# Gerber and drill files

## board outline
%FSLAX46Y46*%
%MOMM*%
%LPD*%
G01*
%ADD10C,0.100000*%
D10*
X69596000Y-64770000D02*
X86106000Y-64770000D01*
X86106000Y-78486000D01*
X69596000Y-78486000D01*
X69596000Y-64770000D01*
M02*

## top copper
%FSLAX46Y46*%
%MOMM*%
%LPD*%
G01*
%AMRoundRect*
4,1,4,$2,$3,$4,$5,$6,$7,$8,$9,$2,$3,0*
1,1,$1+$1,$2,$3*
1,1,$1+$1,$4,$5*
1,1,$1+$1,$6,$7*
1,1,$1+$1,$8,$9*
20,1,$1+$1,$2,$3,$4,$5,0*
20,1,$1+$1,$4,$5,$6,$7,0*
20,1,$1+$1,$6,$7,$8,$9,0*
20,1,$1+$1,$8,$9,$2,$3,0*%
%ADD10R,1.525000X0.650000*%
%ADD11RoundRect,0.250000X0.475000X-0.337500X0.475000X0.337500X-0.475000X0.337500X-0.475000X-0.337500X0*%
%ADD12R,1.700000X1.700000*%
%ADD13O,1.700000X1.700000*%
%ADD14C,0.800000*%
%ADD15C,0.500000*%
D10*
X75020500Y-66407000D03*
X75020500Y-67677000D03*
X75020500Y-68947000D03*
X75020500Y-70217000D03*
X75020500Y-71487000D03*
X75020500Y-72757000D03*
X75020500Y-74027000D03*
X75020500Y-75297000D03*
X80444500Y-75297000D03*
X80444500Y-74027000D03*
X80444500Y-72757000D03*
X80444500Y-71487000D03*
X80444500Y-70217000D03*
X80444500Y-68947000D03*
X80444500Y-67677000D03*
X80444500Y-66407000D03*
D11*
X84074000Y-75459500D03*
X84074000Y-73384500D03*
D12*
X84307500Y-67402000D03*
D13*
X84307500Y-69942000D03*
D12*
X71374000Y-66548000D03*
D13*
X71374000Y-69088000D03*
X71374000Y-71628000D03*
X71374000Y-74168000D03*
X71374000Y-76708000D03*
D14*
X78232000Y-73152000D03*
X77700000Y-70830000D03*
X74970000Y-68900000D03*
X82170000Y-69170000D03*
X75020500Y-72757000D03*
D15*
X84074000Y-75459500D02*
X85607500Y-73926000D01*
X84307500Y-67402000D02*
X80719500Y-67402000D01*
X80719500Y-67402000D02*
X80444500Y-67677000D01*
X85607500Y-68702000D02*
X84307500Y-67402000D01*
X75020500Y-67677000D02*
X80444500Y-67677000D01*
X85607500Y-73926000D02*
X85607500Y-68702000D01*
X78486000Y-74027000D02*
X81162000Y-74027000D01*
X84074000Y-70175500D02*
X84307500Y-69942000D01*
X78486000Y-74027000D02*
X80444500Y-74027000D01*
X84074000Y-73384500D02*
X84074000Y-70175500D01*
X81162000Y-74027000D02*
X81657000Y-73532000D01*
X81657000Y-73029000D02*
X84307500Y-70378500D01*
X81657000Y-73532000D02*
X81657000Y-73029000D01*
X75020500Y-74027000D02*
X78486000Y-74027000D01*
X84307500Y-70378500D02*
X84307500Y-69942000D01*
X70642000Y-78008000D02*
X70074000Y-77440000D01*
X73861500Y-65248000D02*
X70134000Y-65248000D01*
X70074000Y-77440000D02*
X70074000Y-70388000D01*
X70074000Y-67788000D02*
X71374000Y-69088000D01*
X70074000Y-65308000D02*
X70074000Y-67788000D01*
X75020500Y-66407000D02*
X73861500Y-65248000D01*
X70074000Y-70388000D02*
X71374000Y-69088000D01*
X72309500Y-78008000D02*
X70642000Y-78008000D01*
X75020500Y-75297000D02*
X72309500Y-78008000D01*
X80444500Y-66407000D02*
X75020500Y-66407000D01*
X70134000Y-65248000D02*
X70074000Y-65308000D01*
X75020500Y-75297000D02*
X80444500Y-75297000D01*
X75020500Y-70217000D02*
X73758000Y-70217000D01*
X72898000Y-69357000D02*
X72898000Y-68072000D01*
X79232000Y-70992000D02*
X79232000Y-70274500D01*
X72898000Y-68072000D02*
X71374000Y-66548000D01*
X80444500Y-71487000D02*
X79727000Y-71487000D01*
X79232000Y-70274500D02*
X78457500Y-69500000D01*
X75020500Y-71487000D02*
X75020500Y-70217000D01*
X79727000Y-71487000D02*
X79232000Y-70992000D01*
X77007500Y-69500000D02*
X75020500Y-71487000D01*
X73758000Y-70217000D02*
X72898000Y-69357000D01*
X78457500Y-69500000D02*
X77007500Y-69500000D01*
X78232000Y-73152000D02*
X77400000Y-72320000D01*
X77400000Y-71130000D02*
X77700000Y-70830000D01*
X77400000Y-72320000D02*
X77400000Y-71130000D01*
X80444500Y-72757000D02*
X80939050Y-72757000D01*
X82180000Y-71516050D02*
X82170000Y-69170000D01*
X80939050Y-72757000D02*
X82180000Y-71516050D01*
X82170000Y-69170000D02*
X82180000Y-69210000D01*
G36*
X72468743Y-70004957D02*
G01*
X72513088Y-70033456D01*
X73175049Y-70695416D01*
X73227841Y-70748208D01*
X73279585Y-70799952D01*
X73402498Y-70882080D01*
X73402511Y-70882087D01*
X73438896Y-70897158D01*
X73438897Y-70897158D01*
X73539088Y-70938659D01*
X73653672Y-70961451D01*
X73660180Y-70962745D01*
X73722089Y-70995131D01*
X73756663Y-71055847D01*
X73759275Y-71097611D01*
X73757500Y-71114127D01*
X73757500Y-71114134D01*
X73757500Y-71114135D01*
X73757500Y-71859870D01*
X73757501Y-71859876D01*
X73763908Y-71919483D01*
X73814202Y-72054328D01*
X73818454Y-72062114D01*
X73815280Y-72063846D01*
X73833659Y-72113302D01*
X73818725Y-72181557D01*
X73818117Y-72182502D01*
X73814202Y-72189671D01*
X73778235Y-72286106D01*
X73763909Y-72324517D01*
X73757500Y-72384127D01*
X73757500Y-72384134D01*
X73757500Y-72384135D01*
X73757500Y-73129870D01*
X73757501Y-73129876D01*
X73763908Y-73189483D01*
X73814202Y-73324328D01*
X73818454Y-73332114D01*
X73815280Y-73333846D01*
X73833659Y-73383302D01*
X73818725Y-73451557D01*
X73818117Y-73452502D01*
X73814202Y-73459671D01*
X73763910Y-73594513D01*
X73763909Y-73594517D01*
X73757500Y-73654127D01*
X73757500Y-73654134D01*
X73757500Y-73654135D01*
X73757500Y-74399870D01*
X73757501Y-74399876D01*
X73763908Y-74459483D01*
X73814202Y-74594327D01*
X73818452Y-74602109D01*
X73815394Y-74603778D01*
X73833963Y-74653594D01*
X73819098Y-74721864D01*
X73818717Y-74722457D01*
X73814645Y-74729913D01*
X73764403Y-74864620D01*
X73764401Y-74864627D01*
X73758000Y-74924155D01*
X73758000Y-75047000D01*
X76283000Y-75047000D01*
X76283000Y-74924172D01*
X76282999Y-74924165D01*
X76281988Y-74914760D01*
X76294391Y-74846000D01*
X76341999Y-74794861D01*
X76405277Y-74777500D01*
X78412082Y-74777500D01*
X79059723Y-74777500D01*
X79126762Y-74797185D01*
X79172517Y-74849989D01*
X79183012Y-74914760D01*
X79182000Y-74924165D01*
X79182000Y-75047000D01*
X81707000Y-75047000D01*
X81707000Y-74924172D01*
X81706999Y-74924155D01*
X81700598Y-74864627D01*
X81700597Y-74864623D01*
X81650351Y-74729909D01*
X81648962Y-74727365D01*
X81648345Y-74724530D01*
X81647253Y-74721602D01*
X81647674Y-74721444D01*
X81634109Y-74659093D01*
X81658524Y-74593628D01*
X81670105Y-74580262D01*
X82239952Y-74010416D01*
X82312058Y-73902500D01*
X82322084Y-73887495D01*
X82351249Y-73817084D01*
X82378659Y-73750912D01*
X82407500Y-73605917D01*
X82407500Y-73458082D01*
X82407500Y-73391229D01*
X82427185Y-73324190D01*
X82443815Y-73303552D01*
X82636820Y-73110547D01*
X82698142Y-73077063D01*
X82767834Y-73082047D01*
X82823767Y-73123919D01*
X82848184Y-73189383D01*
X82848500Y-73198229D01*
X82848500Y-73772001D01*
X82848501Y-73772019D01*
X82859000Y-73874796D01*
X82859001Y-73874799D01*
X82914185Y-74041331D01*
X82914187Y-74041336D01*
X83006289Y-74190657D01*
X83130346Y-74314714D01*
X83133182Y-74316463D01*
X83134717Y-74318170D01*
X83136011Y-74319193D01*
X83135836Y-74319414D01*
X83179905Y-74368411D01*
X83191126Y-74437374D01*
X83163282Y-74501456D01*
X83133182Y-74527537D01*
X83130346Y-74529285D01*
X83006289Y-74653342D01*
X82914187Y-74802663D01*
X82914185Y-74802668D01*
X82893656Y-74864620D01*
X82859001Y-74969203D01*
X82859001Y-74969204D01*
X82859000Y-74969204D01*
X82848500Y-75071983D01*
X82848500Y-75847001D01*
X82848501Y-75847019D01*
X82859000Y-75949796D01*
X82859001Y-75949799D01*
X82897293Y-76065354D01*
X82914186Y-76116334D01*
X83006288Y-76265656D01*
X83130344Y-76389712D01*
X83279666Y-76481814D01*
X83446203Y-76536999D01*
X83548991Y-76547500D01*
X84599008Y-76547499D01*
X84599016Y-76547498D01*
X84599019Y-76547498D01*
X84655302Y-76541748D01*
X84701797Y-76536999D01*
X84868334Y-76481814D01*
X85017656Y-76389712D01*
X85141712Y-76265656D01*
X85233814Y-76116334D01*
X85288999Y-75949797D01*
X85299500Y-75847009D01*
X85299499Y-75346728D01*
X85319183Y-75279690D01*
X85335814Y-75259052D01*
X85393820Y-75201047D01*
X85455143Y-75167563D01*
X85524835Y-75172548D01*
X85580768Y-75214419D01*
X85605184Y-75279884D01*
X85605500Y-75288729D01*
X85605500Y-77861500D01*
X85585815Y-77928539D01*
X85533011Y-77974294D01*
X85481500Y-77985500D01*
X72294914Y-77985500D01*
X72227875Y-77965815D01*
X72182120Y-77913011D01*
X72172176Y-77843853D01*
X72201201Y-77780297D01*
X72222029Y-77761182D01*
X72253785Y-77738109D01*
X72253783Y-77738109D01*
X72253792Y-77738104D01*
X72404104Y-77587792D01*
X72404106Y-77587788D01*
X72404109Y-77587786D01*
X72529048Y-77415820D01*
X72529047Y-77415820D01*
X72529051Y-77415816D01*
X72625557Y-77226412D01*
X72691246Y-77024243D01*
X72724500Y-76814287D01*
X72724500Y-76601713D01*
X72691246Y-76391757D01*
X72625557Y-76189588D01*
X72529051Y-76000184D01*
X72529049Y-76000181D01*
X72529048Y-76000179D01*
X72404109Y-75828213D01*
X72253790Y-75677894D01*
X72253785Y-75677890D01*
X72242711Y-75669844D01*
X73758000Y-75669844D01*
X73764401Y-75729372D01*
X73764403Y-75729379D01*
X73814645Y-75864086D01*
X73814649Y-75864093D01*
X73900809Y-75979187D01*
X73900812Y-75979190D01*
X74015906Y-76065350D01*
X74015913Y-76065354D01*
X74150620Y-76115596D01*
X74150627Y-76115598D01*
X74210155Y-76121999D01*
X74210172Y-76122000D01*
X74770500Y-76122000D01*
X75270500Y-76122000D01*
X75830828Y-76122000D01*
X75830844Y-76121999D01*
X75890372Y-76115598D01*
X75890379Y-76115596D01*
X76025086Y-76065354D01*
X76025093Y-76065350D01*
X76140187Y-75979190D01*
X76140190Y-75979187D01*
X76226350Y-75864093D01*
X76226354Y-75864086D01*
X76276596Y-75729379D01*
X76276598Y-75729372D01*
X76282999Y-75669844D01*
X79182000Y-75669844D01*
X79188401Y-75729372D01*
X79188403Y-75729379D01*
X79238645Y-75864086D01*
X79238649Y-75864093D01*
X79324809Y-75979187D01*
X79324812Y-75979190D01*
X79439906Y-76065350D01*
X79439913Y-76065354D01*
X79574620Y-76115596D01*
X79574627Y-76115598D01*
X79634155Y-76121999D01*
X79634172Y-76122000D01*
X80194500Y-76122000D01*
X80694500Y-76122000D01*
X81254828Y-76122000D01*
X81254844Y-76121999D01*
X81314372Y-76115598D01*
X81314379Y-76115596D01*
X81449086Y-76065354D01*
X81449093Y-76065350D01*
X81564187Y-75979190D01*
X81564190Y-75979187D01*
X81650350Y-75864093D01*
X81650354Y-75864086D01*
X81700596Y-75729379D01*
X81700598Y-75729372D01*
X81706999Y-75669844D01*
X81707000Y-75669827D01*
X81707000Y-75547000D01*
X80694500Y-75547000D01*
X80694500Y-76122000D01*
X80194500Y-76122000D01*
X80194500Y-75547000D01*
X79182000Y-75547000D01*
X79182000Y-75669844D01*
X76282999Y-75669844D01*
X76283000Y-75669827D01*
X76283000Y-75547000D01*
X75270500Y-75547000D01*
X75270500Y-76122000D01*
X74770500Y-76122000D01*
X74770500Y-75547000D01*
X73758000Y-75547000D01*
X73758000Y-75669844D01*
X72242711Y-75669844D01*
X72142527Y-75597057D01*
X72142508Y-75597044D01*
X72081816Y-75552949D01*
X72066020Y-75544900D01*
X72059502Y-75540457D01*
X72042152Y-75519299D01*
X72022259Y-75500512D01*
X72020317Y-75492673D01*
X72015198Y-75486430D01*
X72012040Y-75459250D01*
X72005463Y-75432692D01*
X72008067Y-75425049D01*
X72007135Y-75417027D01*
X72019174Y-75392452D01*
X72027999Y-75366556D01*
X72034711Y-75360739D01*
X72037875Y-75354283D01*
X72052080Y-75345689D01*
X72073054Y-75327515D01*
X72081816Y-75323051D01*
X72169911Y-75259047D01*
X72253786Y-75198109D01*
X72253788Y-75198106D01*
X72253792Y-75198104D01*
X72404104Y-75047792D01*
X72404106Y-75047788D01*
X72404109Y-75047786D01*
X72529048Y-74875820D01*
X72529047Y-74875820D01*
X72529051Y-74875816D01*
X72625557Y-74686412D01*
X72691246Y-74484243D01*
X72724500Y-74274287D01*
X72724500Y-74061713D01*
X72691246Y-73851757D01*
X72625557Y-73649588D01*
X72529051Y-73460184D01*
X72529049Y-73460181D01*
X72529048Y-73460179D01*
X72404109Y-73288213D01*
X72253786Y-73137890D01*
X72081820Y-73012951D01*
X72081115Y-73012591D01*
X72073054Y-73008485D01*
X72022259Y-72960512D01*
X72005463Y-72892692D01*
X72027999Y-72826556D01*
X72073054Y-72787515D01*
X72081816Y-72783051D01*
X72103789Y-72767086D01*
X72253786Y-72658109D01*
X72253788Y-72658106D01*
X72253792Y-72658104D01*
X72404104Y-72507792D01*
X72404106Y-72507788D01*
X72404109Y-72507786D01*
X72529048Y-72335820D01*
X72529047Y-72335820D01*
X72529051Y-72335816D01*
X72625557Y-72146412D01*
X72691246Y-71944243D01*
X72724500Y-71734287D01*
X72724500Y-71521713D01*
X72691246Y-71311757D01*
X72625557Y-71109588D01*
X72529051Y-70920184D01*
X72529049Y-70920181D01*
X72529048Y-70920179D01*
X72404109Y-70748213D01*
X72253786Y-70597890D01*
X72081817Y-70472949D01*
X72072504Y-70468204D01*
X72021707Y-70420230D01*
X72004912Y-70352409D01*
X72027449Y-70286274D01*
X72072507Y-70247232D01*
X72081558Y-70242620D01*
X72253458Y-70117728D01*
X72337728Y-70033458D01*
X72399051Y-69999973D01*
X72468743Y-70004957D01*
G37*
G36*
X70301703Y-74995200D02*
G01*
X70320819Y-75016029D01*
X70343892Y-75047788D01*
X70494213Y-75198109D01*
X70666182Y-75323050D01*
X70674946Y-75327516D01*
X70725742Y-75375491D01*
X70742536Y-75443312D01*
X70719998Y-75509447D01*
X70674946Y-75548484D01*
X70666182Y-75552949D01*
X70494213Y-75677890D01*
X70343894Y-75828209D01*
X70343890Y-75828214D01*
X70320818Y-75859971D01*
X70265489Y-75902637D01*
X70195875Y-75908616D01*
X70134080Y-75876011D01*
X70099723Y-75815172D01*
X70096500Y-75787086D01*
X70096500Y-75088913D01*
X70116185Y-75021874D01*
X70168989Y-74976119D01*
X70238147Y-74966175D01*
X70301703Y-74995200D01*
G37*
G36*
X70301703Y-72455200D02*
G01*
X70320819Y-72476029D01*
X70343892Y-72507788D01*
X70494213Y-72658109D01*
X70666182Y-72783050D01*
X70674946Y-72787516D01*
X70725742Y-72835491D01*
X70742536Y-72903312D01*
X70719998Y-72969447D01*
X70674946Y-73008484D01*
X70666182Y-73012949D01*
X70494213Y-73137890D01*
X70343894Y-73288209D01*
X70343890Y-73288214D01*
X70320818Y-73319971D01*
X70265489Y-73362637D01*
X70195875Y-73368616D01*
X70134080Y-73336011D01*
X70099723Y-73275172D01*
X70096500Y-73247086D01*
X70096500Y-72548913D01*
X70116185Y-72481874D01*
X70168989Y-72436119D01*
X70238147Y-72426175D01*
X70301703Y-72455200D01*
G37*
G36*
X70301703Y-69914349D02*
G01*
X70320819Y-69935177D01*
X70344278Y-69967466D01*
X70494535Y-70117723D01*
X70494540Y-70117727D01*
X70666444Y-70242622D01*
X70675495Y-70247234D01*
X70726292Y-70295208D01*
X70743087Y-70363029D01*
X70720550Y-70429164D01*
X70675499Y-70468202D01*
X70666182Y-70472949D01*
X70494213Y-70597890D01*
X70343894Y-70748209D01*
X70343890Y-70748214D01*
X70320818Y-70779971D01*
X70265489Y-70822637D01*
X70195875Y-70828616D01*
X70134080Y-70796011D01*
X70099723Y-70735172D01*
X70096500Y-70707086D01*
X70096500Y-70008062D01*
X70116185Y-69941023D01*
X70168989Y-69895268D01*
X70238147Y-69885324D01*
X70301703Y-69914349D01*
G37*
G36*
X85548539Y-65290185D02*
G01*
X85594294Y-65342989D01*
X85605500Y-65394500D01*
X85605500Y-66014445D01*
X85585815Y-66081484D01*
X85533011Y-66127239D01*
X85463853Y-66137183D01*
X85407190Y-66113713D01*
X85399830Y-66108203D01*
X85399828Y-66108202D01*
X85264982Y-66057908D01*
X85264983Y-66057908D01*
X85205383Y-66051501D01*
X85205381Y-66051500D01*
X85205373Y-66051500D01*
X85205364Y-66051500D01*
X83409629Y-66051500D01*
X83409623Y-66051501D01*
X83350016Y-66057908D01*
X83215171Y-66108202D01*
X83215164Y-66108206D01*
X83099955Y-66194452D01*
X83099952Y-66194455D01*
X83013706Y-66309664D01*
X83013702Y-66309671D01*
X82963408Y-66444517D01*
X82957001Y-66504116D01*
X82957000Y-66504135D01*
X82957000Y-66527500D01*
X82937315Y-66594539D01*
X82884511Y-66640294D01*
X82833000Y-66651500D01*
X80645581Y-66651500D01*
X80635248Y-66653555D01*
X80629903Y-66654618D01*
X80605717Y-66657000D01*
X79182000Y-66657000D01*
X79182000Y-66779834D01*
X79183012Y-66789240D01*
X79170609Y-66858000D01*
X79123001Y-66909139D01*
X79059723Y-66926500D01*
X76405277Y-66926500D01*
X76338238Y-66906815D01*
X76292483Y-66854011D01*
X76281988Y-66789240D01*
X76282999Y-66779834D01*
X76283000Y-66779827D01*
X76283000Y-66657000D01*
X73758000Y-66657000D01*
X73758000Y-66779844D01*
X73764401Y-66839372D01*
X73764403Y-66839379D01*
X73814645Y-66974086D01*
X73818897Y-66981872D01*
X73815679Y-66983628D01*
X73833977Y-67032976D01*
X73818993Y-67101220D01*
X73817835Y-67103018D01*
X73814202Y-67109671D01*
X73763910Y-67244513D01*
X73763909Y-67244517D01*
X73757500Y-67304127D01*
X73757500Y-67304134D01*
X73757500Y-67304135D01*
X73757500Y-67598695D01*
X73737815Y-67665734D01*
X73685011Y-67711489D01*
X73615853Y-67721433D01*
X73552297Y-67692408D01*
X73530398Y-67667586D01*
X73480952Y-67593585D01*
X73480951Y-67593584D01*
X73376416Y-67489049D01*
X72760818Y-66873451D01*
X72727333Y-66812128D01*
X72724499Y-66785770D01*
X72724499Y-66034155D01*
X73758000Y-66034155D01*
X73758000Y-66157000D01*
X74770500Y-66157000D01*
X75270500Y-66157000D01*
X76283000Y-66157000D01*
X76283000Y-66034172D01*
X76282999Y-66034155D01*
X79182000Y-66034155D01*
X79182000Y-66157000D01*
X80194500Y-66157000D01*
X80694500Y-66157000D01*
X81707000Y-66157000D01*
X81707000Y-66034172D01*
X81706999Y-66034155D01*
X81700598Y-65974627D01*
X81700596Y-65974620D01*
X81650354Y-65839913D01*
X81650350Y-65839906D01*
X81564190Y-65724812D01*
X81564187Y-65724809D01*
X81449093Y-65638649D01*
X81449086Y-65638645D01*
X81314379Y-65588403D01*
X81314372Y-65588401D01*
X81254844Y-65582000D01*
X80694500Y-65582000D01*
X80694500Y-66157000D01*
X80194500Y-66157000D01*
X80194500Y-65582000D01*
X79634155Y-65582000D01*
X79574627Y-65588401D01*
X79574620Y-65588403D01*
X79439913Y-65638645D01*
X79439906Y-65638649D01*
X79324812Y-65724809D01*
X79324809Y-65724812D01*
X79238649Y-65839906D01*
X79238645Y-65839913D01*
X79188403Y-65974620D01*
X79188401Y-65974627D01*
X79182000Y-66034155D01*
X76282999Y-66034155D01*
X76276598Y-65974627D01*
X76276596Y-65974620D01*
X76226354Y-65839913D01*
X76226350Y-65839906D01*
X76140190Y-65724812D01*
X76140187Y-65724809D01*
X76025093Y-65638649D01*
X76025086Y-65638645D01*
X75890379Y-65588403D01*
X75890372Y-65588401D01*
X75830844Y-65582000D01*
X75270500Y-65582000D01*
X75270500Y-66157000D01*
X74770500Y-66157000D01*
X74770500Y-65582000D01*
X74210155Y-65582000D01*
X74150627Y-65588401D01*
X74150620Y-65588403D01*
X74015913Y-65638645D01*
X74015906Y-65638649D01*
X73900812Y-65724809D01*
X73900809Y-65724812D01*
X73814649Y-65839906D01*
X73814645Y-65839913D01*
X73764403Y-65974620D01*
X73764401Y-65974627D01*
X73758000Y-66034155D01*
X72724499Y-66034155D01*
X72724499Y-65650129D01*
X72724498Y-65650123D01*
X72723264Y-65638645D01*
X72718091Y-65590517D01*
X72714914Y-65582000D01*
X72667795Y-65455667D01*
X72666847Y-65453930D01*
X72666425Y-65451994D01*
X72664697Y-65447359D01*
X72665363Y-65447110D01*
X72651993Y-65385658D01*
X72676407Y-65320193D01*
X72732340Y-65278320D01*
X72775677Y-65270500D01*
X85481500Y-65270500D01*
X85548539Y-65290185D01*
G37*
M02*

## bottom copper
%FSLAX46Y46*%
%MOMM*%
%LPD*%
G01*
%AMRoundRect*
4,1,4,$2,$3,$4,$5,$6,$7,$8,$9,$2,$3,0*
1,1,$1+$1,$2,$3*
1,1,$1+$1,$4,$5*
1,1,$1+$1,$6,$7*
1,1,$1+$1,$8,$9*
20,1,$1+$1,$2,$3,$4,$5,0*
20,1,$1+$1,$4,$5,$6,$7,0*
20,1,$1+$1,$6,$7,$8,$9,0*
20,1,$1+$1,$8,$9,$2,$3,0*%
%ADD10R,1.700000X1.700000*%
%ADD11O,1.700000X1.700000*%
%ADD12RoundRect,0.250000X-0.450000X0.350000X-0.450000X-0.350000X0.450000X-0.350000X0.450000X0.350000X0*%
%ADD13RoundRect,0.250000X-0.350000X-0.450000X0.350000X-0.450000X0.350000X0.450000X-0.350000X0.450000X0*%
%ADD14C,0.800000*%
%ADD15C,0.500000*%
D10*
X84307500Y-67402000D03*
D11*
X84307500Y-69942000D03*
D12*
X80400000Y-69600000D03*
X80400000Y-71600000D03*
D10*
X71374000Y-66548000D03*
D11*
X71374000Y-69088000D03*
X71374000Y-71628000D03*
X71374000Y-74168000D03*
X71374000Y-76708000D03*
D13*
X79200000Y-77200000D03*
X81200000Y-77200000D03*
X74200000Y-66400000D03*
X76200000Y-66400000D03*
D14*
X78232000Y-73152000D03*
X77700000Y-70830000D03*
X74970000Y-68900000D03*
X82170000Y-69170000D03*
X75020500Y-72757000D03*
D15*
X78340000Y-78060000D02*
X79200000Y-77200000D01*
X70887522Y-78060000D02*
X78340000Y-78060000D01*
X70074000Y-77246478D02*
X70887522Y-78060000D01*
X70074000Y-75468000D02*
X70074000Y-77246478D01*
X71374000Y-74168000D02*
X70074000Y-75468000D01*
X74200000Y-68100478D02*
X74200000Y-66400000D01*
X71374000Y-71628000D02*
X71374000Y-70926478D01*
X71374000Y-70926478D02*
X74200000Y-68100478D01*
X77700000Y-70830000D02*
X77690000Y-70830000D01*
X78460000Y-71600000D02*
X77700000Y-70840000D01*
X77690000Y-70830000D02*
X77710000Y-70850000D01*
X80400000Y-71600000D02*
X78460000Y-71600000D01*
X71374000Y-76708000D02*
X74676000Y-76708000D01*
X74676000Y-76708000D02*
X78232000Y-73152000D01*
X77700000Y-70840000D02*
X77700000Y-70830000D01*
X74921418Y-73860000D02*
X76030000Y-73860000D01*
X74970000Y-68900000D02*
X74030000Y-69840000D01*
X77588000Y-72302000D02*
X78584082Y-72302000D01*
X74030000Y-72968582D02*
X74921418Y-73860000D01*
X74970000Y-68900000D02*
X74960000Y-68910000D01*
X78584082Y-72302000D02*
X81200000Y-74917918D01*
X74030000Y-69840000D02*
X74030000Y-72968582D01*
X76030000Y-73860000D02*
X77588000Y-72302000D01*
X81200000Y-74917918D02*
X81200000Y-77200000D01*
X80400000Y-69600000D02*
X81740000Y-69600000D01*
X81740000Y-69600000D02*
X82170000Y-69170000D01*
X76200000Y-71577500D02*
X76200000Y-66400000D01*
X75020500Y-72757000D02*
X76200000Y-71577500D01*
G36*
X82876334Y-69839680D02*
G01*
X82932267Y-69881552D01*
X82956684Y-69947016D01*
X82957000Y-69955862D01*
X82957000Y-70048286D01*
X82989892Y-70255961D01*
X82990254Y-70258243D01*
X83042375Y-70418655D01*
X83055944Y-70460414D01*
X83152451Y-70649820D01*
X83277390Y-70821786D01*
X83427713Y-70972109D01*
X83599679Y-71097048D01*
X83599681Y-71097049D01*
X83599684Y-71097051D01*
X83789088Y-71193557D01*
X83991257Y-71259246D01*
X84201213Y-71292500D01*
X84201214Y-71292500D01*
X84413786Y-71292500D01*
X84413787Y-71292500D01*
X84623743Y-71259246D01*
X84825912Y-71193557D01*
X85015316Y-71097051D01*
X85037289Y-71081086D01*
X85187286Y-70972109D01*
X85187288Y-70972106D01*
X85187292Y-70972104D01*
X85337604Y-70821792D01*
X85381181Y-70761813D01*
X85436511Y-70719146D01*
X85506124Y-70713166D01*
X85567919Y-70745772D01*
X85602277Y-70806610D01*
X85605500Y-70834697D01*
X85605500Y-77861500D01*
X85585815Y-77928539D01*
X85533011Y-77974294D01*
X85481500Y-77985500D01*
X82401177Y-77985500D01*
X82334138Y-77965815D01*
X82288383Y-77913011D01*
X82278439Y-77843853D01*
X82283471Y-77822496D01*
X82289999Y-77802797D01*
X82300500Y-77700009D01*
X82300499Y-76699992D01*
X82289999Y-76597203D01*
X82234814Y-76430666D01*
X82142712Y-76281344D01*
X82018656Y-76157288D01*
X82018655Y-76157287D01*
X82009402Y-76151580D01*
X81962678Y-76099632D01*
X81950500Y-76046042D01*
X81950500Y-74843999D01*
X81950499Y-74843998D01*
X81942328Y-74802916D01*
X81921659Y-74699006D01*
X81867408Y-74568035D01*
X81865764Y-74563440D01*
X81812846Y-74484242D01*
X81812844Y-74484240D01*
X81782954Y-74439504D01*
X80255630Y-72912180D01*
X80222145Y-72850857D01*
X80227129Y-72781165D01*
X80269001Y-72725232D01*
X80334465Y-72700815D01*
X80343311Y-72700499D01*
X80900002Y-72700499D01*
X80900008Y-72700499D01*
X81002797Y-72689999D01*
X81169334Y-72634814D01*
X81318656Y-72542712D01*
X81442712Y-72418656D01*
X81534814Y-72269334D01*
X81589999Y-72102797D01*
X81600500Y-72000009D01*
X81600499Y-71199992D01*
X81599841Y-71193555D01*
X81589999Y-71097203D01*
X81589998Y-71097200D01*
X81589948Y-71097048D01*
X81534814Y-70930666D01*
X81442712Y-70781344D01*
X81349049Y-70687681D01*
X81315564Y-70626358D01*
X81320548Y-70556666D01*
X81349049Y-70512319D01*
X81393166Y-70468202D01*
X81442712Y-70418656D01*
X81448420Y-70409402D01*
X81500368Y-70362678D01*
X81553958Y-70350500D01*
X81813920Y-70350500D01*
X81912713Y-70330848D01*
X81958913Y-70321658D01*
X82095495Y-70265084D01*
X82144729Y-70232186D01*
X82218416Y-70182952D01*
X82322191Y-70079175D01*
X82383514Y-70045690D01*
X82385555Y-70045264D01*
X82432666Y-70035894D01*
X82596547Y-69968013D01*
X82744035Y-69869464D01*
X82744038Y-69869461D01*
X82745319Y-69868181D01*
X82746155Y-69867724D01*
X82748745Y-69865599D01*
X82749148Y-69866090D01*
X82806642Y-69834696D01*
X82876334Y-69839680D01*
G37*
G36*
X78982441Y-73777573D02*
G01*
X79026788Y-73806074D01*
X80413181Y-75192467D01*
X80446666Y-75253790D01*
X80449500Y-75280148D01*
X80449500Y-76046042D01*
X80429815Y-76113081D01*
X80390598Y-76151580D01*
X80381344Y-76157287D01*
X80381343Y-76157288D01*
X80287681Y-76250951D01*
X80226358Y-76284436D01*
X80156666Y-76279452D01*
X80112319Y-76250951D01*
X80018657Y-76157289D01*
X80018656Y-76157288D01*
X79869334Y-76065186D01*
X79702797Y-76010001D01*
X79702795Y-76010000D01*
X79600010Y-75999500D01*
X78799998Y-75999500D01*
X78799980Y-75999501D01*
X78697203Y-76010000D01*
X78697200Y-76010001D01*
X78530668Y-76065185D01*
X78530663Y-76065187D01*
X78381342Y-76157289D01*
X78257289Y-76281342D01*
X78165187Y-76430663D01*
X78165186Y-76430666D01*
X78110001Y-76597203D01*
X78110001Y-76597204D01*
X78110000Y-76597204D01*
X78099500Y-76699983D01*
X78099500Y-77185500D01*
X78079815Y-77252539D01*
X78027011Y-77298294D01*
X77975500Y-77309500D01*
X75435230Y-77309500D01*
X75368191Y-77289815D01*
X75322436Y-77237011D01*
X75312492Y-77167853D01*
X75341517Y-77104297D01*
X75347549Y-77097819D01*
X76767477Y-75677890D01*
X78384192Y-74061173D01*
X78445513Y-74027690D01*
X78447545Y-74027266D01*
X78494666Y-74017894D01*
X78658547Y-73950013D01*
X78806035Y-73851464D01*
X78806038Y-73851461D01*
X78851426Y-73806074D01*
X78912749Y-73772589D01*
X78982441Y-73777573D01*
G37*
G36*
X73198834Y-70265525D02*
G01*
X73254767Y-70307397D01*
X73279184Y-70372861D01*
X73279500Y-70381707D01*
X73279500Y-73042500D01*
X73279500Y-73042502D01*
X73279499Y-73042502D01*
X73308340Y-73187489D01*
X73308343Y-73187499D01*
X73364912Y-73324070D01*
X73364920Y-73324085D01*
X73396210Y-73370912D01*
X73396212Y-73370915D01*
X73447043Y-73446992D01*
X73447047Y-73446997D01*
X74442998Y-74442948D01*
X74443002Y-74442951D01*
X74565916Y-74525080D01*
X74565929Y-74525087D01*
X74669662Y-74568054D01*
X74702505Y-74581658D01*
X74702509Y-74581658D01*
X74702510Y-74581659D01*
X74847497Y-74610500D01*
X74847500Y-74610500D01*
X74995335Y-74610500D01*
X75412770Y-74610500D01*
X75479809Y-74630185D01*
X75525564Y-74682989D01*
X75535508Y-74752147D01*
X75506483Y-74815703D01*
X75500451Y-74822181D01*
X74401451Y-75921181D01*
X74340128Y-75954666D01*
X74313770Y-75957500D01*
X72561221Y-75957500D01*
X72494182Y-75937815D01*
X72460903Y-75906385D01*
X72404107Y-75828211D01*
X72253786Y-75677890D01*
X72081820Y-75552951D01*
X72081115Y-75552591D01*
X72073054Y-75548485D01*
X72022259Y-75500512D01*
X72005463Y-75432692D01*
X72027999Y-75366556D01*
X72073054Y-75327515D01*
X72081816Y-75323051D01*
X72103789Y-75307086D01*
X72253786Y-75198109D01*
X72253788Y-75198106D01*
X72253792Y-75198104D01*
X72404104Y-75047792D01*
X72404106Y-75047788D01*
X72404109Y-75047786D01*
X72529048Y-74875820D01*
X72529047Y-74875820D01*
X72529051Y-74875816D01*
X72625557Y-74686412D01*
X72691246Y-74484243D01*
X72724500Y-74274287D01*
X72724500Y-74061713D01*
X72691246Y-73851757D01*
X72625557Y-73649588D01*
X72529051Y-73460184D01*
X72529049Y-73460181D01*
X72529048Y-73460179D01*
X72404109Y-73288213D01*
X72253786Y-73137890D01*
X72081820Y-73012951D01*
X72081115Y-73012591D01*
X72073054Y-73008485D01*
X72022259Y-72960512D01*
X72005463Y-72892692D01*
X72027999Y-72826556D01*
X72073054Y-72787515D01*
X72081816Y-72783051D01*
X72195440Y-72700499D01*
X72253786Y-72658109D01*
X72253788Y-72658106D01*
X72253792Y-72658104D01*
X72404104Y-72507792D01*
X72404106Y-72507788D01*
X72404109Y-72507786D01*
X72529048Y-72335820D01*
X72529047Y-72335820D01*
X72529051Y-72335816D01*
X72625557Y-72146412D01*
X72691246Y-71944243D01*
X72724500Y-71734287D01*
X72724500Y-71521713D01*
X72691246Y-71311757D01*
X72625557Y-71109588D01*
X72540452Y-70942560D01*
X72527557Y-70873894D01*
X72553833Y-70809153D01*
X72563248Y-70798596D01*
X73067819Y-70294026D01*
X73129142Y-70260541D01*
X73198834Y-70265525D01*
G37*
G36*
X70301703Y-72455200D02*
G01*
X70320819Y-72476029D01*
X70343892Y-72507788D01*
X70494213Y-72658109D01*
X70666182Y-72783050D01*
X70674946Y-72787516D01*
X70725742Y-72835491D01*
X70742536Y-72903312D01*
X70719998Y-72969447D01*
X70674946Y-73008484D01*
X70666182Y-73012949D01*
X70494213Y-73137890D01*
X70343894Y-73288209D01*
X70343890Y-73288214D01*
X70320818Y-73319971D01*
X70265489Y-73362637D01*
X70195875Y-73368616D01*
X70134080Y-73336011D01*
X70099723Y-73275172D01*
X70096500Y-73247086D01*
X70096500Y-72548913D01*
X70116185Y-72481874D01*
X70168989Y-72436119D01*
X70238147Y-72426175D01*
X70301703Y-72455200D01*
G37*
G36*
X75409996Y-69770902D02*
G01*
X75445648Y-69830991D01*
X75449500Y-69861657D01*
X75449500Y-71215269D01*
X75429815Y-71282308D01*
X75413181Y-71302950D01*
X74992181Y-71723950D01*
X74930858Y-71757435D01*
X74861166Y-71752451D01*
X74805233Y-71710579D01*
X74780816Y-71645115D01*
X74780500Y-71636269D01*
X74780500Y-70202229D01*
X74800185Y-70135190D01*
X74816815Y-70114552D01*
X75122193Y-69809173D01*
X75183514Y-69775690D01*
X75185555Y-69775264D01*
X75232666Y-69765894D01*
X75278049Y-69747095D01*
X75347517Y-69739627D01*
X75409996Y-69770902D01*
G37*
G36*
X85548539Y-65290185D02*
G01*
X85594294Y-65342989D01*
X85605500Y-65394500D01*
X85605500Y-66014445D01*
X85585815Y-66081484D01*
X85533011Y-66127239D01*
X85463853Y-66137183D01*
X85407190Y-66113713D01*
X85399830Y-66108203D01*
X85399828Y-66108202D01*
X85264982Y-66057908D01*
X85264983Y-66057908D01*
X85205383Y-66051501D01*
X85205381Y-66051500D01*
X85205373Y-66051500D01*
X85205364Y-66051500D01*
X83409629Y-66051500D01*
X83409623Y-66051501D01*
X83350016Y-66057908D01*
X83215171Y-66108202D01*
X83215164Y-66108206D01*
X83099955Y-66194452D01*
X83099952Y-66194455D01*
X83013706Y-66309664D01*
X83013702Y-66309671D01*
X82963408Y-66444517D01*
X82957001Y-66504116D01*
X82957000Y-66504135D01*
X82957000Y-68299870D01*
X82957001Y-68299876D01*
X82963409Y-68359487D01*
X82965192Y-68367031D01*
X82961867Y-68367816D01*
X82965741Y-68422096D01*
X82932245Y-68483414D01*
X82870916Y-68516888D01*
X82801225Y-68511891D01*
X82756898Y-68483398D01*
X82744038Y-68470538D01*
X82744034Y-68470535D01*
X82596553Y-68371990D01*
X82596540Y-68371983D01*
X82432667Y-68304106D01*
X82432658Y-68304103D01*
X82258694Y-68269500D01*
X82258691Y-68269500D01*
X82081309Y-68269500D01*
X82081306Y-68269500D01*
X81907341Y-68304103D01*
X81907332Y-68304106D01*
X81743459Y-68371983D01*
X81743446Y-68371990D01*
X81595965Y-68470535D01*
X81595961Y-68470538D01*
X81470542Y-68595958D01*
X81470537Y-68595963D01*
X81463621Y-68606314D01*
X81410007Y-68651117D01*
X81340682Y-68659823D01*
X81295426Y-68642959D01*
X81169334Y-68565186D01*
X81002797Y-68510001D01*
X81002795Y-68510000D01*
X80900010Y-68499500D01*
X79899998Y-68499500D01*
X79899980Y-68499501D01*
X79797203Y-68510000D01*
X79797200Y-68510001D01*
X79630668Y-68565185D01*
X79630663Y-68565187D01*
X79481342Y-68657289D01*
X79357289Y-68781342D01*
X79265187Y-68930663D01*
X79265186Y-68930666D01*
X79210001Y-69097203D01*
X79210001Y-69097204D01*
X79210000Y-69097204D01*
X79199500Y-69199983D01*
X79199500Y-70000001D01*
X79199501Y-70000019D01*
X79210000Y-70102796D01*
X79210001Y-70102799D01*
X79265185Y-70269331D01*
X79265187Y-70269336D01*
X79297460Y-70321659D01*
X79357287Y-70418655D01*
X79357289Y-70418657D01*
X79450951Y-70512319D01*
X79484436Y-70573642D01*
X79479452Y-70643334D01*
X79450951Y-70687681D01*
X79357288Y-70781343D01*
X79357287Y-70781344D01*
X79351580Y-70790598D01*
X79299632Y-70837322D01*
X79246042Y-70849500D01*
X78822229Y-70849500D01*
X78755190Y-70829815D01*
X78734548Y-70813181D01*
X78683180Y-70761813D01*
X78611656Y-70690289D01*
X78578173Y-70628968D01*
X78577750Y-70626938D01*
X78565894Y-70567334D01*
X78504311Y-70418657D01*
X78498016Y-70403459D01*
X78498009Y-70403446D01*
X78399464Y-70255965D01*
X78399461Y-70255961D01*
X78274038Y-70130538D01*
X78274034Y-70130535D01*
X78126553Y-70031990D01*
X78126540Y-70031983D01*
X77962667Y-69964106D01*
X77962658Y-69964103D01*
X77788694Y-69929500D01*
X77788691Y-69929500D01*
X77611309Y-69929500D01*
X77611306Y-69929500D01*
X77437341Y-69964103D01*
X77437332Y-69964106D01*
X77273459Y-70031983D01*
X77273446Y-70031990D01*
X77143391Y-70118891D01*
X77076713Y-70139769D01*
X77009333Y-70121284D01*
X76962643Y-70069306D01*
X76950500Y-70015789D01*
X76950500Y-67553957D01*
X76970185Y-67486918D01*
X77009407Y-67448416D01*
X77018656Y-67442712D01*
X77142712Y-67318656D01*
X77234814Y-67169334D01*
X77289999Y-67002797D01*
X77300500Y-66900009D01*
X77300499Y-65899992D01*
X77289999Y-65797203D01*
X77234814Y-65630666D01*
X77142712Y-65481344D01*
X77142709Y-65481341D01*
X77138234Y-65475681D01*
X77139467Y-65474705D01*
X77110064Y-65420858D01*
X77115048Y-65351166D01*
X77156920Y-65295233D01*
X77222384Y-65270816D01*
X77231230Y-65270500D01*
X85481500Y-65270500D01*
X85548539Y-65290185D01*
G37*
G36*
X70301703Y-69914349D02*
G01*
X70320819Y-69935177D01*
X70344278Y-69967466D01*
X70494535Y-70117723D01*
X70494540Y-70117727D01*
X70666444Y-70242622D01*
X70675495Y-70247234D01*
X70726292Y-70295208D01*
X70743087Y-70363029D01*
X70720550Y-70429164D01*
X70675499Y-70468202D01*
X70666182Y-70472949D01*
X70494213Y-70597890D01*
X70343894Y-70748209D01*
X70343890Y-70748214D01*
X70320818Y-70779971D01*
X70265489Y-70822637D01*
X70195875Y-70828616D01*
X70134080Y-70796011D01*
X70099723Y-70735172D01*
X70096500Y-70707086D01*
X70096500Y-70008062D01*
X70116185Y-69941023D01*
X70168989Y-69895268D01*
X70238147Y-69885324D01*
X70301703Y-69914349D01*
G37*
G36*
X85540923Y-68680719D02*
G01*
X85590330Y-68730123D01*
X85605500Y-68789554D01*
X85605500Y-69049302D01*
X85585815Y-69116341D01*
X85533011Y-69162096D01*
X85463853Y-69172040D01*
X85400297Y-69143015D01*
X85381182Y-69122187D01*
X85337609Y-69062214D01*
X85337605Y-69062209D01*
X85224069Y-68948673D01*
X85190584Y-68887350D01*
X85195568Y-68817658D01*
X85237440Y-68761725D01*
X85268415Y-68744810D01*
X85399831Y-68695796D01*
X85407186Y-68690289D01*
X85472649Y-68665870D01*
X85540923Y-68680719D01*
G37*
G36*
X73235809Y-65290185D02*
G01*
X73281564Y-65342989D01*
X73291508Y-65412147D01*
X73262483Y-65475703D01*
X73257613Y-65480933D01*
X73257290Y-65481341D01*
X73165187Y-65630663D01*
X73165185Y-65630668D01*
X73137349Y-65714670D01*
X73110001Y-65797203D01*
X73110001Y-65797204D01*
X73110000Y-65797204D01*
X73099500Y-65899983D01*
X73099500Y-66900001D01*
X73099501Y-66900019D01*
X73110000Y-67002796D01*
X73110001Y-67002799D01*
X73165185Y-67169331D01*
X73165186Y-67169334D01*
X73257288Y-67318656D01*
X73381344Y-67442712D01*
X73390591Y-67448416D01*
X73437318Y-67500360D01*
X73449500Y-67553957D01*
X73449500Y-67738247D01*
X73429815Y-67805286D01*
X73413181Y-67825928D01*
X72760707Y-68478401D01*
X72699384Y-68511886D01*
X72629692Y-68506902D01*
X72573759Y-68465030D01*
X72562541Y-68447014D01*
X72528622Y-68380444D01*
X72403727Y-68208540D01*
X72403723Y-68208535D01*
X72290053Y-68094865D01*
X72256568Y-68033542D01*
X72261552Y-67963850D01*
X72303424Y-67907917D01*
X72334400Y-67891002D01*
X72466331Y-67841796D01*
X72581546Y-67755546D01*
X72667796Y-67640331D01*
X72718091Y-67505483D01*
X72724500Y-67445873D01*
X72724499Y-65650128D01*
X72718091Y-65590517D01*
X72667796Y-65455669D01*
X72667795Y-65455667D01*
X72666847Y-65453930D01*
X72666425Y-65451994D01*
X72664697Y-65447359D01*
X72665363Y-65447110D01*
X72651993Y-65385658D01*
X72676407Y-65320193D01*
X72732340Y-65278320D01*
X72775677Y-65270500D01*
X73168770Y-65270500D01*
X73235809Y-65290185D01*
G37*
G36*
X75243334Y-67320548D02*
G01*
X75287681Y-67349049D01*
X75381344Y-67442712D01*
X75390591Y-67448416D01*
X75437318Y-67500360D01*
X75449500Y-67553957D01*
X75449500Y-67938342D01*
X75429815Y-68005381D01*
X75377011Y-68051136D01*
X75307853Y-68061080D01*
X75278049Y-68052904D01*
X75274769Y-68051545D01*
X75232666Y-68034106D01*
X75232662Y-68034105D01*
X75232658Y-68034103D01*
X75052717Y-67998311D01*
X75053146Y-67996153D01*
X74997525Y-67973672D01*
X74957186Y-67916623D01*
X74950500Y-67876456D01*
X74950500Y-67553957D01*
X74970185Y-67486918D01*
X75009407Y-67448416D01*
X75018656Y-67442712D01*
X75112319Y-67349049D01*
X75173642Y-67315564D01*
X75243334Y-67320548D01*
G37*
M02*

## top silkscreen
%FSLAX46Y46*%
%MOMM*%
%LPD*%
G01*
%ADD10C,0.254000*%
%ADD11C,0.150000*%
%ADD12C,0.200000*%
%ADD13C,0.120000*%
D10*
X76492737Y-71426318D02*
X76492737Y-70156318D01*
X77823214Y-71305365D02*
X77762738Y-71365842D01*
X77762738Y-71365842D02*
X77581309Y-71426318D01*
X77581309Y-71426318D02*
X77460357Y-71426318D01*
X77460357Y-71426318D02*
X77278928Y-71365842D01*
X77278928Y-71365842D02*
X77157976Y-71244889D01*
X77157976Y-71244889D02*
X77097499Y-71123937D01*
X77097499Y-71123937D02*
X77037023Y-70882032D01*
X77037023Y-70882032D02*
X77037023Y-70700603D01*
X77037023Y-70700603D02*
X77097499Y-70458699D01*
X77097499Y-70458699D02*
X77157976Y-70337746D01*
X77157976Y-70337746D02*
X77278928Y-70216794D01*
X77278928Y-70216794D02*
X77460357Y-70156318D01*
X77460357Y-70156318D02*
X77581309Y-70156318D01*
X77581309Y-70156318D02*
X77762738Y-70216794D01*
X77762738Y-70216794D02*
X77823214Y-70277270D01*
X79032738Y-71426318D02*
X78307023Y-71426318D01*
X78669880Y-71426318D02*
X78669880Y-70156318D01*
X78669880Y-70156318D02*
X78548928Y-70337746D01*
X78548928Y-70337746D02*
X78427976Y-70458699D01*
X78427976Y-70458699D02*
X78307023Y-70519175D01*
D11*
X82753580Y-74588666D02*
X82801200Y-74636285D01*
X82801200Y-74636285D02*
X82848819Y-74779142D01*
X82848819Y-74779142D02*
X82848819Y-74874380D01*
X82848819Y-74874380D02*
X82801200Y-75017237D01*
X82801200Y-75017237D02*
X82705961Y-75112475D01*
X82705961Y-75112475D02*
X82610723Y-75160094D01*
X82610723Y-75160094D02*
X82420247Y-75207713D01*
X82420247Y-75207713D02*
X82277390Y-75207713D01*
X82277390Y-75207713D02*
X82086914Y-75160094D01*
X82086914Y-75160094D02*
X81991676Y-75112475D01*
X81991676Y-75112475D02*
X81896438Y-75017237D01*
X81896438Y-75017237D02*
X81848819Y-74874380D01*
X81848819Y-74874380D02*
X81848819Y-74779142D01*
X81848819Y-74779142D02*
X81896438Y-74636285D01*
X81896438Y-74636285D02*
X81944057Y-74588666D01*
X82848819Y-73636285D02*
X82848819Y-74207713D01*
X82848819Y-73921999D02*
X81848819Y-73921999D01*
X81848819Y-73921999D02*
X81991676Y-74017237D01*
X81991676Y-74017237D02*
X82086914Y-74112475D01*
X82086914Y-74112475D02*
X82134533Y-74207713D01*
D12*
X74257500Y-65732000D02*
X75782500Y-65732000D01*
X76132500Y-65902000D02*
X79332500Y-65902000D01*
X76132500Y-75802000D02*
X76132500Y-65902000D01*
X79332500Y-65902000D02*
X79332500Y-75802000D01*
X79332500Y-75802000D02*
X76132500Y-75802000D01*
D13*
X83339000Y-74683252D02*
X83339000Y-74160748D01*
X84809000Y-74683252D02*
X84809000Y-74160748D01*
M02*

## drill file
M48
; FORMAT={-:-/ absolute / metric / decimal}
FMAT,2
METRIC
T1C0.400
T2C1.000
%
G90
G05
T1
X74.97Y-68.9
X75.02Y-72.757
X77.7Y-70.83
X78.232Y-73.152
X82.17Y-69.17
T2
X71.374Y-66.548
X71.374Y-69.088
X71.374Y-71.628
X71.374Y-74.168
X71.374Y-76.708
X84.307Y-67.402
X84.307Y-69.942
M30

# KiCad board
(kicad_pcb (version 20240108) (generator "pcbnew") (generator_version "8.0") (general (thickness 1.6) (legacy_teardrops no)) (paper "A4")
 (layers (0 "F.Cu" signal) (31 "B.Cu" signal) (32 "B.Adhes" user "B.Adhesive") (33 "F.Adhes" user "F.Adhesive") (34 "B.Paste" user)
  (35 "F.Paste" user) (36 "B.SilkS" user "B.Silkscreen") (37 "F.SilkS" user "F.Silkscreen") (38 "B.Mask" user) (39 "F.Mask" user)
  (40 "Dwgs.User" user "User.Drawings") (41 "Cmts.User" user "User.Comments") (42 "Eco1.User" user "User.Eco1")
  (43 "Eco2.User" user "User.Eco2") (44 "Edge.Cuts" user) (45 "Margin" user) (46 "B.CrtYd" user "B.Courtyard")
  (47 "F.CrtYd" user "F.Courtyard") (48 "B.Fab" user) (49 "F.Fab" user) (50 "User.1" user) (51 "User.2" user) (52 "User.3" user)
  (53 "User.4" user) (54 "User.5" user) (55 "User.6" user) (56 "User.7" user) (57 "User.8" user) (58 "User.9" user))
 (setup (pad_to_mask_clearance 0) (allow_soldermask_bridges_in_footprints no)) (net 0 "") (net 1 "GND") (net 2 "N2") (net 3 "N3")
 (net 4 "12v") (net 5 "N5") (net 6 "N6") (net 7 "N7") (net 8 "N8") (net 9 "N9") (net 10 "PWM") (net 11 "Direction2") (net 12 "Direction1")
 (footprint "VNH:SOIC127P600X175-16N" (layer "F.Cu") (at 77.7325 70.852)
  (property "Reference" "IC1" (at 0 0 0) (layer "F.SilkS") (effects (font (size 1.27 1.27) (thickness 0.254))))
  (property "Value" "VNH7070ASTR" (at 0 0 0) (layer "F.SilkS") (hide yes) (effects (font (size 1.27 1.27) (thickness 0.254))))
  (fp_line (start -3.475 -5.12) (end -1.95 -5.12) (stroke (width 0.2) (type solid)) (layer "F.SilkS"))
  (fp_line (start -1.6 -4.95) (end 1.6 -4.95) (stroke (width 0.2) (type solid)) (layer "F.SilkS"))
  (fp_line (start -1.6 4.95) (end -1.6 -4.95) (stroke (width 0.2) (type solid)) (layer "F.SilkS"))
  (fp_line (start 1.6 -4.95) (end 1.6 4.95) (stroke (width 0.2) (type solid)) (layer "F.SilkS"))
  (fp_line (start 1.6 4.95) (end -1.6 4.95) (stroke (width 0.2) (type solid)) (layer "F.SilkS"))
  (pad "1" smd rect (at -2.712 -4.445 90) (size 0.65 1.525) (layers "F.Cu" "F.Paste" "F.Mask") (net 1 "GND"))
  (pad "2" smd rect (at -2.712 -3.175 90) (size 0.65 1.525) (layers "F.Cu" "F.Paste" "F.Mask") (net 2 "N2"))
  (pad "3" smd rect (at -2.712 -1.905 90) (size 0.65 1.525) (layers "F.Cu" "F.Paste" "F.Mask") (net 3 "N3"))
  (pad "4" smd rect (at -2.712 -0.635 90) (size 0.65 1.525) (layers "F.Cu" "F.Paste" "F.Mask") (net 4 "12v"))
  (pad "5" smd rect (at -2.712 0.635 90) (size 0.65 1.525) (layers "F.Cu" "F.Paste" "F.Mask") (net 4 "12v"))
  (pad "6" smd rect (at -2.712 1.905 90) (size 0.65 1.525) (layers "F.Cu" "F.Paste" "F.Mask") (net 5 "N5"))
  (pad "7" smd rect (at -2.712 3.175 90) (size 0.65 1.525) (layers "F.Cu" "F.Paste" "F.Mask") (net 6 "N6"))
  (pad "8" smd rect (at -2.712 4.445 90) (size 0.65 1.525) (layers "F.Cu" "F.Paste" "F.Mask") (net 1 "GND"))
  (pad "9" smd rect (at 2.712 4.445 90) (size 0.65 1.525) (layers "F.Cu" "F.Paste" "F.Mask") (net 1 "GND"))
  (pad "10" smd rect (at 2.712 3.175 90) (size 0.65 1.525) (layers "F.Cu" "F.Paste" "F.Mask") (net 6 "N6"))
  (pad "11" smd rect (at 2.712 1.905 90) (size 0.65 1.525) (layers "F.Cu" "F.Paste" "F.Mask") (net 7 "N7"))
  (pad "12" smd rect (at 2.712 0.635 90) (size 0.65 1.525) (layers "F.Cu" "F.Paste" "F.Mask") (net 4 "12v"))
  (pad "13" smd rect (at 2.712 -0.635 90) (size 0.65 1.525) (layers "F.Cu" "F.Paste" "F.Mask") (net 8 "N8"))
  (pad "14" smd rect (at 2.712 -1.905 90) (size 0.65 1.525) (layers "F.Cu" "F.Paste" "F.Mask") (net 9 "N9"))
  (pad "15" smd rect (at 2.712 -3.175 90) (size 0.65 1.525) (layers "F.Cu" "F.Paste" "F.Mask") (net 2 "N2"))
  (pad "16" smd rect (at 2.712 -4.445 90) (size 0.65 1.525) (layers "F.Cu" "F.Paste" "F.Mask") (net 1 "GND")))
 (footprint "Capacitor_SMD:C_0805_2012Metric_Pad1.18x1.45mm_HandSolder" (layer "F.Cu") (at 84.074 74.422 90)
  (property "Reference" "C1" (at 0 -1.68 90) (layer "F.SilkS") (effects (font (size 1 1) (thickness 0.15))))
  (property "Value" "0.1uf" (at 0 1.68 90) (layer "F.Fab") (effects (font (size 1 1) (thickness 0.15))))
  (fp_line (start -0.261252 -0.735) (end 0.261252 -0.735) (stroke (width 0.12) (type solid)) (layer "F.SilkS"))
  (fp_line (start -0.261252 0.735) (end 0.261252 0.735) (stroke (width 0.12) (type solid)) (layer "F.SilkS"))
  (pad "1" smd roundrect (at -1.0375 0 90) (size 1.175 1.45) (layers "F.Cu" "F.Paste" "F.Mask") (roundrect_rratio 0.2127659574) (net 2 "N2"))
  (pad "2" smd roundrect (at 1.0375 0 90) (size 1.175 1.45) (layers "F.Cu" "F.Paste" "F.Mask") (roundrect_rratio 0.2127659574) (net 6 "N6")))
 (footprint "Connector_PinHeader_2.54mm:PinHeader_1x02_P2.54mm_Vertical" (layer "B.Cu") (at 84.3075 67.402 180)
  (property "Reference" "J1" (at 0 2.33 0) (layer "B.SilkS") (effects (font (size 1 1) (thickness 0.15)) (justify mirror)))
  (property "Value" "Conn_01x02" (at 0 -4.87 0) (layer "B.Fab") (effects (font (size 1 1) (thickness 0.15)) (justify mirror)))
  (pad "1" thru_hole rect (at 0 0 180) (size 1.7 1.7) (drill 1) (layers "*.Cu" "*.Mask") (remove_unused_layers no) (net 2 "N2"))
  (pad "2" thru_hole oval (at 0 -2.54 180) (size 1.7 1.7) (drill 1) (layers "*.Cu" "*.Mask") (remove_unused_layers no) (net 6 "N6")))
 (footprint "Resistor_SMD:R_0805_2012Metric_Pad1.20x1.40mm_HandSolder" (layer "B.Cu") (at 80.4 70.6 -90)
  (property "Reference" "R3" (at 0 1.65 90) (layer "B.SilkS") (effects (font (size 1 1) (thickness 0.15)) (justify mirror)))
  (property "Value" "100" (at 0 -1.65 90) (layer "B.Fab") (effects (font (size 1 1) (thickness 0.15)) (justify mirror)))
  (pad "1" smd roundrect (at -1 0 270) (size 1.2 1.4) (layers "B.Cu" "B.Paste" "B.Mask") (roundrect_rratio 0.2083333333) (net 7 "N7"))
  (pad "2" smd roundrect (at 1 0 270) (size 1.2 1.4) (layers "B.Cu" "B.Paste" "B.Mask") (roundrect_rratio 0.2083333333) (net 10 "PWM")))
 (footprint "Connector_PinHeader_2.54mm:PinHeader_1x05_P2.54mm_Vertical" (layer "B.Cu") (at 71.374 66.548 180)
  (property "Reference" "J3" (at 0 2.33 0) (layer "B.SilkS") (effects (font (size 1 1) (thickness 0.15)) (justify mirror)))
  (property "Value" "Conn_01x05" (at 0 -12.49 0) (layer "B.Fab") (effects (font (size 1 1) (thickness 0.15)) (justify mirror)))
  (pad "1" thru_hole rect (at 0 0 180) (size 1.7 1.7) (drill 1) (layers "*.Cu" "*.Mask") (remove_unused_layers no) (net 4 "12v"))
  (pad "2" thru_hole oval (at 0 -2.54 180) (size 1.7 1.7) (drill 1) (layers "*.Cu" "*.Mask") (remove_unused_layers no) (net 1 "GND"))
  (pad "3" thru_hole oval (at 0 -5.08 180) (size 1.7 1.7) (drill 1) (layers "*.Cu" "*.Mask") (remove_unused_layers no) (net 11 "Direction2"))
  (pad "4" thru_hole oval (at 0 -7.62 180) (size 1.7 1.7) (drill 1) (layers "*.Cu" "*.Mask") (remove_unused_layers no) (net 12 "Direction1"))
  (pad "5" thru_hole oval (at 0 -10.16 180) (size 1.7 1.7) (drill 1) (layers "*.Cu" "*.Mask") (remove_unused_layers no) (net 10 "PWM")))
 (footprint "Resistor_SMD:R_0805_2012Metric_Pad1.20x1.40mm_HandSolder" (layer "B.Cu") (at 80.2 77.2)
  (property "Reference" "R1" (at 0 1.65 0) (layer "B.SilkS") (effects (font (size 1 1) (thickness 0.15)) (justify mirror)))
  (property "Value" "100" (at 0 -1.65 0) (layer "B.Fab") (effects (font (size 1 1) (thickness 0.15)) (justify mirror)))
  (pad "1" smd roundrect (at -1 0) (size 1.2 1.4) (layers "B.Cu" "B.Paste" "B.Mask") (roundrect_rratio 0.2083333333) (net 12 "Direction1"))
  (pad "2" smd roundrect (at 1 0) (size 1.2 1.4) (layers "B.Cu" "B.Paste" "B.Mask") (roundrect_rratio 0.2083333333) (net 3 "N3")))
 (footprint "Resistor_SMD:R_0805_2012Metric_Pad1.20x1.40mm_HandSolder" (layer "B.Cu") (at 75.2 66.4)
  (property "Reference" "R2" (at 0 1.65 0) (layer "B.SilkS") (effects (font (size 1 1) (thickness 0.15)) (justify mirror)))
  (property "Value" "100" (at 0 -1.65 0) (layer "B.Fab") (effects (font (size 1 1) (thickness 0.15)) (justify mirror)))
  (pad "1" smd roundrect (at -1 0) (size 1.2 1.4) (layers "B.Cu" "B.Paste" "B.Mask") (roundrect_rratio 0.2083333333) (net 11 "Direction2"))
  (pad "2" smd roundrect (at 1 0) (size 1.2 1.4) (layers "B.Cu" "B.Paste" "B.Mask") (roundrect_rratio 0.2083333333) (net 5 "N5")))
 (gr_rect (start 69.596 64.77) (end 86.106 78.486) (stroke (width 0.1) (type default)) (fill none) (layer "Edge.Cuts"))
 (segment (start 84.074 75.4595) (end 85.6075 73.926) (width 0.5) (layer "F.Cu") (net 2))
 (segment (start 84.3075 67.402) (end 80.7195 67.402) (width 0.5) (layer "F.Cu") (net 2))
 (segment (start 80.7195 67.402) (end 80.4445 67.677) (width 0.5) (layer "F.Cu") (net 2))
 (segment (start 85.6075 68.702) (end 84.3075 67.402) (width 0.5) (layer "F.Cu") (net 2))
 (segment (start 75.0205 67.677) (end 80.4445 67.677) (width 0.5) (layer "F.Cu") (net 2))
 (segment (start 85.6075 73.926) (end 85.6075 68.702) (width 0.5) (layer "F.Cu") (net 2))
 (segment (start 78.486 74.027) (end 81.162 74.027) (width 0.5) (layer "F.Cu") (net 6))
 (segment (start 84.074 70.1755) (end 84.3075 69.942) (width 0.5) (layer "F.Cu") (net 6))
 (segment (start 78.486 74.027) (end 80.4445 74.027) (width 0.5) (layer "F.Cu") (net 6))
 (segment (start 84.074 73.3845) (end 84.074 70.1755) (width 0.5) (layer "F.Cu") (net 6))
 (segment (start 81.162 74.027) (end 81.657 73.532) (width 0.5) (layer "F.Cu") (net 6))
 (segment (start 81.657 73.029) (end 84.3075 70.3785) (width 0.5) (layer "F.Cu") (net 6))
 (segment (start 81.657 73.532) (end 81.657 73.029) (width 0.5) (layer "F.Cu") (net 6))
 (segment (start 75.0205 74.027) (end 78.486 74.027) (width 0.5) (layer "F.Cu") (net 6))
 (segment (start 84.3075 70.3785) (end 84.3075 69.942) (width 0.5) (layer "F.Cu") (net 6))
 (segment (start 70.642 78.008) (end 70.074 77.44) (width 0.5) (layer "F.Cu") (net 1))
 (segment (start 73.8615 65.248) (end 70.134 65.248) (width 0.5) (layer "F.Cu") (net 1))
 (segment (start 70.074 77.44) (end 70.074 70.388) (width 0.5) (layer "F.Cu") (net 1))
 (segment (start 70.074 67.788) (end 71.374 69.088) (width 0.5) (layer "F.Cu") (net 1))
 (segment (start 70.074 65.308) (end 70.074 67.788) (width 0.5) (layer "F.Cu") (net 1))
 (segment (start 75.0205 66.407) (end 73.8615 65.248) (width 0.5) (layer "F.Cu") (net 1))
 (segment (start 70.074 70.388) (end 71.374 69.088) (width 0.5) (layer "F.Cu") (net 1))
 (segment (start 72.3095 78.008) (end 70.642 78.008) (width 0.5) (layer "F.Cu") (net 1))
 (segment (start 75.0205 75.297) (end 72.3095 78.008) (width 0.5) (layer "F.Cu") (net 1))
 (segment (start 80.4445 66.407) (end 75.0205 66.407) (width 0.5) (layer "F.Cu") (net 1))
 (segment (start 70.134 65.248) (end 70.074 65.308) (width 0.5) (layer "F.Cu") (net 1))
 (segment (start 75.0205 75.297) (end 80.4445 75.297) (width 0.5) (layer "F.Cu") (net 1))
 (segment (start 78.34 78.06) (end 79.2 77.2) (width 0.5) (layer "B.Cu") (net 12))
 (segment (start 70.887522 78.06) (end 78.34 78.06) (width 0.5) (layer "B.Cu") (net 12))
 (segment (start 70.074 77.246478) (end 70.887522 78.06) (width 0.5) (layer "B.Cu") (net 12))
 (segment (start 70.074 75.468) (end 70.074 77.246478) (width 0.5) (layer "B.Cu") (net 12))
 (segment (start 71.374 74.168) (end 70.074 75.468) (width 0.5) (layer "B.Cu") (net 12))
 (segment (start 75.0205 70.217) (end 73.758 70.217) (width 0.5) (layer "F.Cu") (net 4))
 (segment (start 72.898 69.357) (end 72.898 68.072) (width 0.5) (layer "F.Cu") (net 4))
 (segment (start 79.232 70.992) (end 79.232 70.2745) (width 0.5) (layer "F.Cu") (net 4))
 (segment (start 72.898 68.072) (end 71.374 66.548) (width 0.5) (layer "F.Cu") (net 4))
 (segment (start 80.4445 71.487) (end 79.727 71.487) (width 0.5) (layer "F.Cu") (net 4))
 (segment (start 79.232 70.2745) (end 78.4575 69.5) (width 0.5) (layer "F.Cu") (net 4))
 (segment (start 75.0205 71.487) (end 75.0205 70.217) (width 0.5) (layer "F.Cu") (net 4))
 (segment (start 79.727 71.487) (end 79.232 70.992) (width 0.5) (layer "F.Cu") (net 4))
 (segment (start 77.0075 69.5) (end 75.0205 71.487) (width 0.5) (layer "F.Cu") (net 4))
 (segment (start 73.758 70.217) (end 72.898 69.357) (width 0.5) (layer "F.Cu") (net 4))
 (segment (start 78.4575 69.5) (end 77.0075 69.5) (width 0.5) (layer "F.Cu") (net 4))
 (segment (start 74.2 68.100478) (end 74.2 66.4) (width 0.5) (layer "B.Cu") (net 11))
 (segment (start 71.374 71.628) (end 71.374 70.926478) (width 0.5) (layer "B.Cu") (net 11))
 (segment (start 71.374 70.926478) (end 74.2 68.100478) (width 0.5) (layer "B.Cu") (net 11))
 (segment (start 78.232 73.152) (end 77.4 72.32) (width 0.5) (layer "F.Cu") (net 10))
 (segment (start 77.4 71.13) (end 77.7 70.83) (width 0.5) (layer "F.Cu") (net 10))
 (segment (start 77.4 72.32) (end 77.4 71.13) (width 0.5) (layer "F.Cu") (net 10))
 (via (at 78.232 73.152) (size 0.8) (drill 0.4) (layers "F.Cu" "B.Cu") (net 10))
 (via (at 77.7 70.83) (size 0.8) (drill 0.4) (layers "F.Cu" "B.Cu") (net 10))
 (segment (start 77.7 70.83) (end 77.69 70.83) (width 0.5) (layer "B.Cu") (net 10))
 (segment (start 78.46 71.6) (end 77.7 70.84) (width 0.5) (layer "B.Cu") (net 10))
 (segment (start 77.69 70.83) (end 77.71 70.85) (width 0.5) (layer "B.Cu") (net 10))
 (segment (start 80.4 71.6) (end 78.46 71.6) (width 0.5) (layer "B.Cu") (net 10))
 (segment (start 71.374 76.708) (end 74.676 76.708) (width 0.5) (layer "B.Cu") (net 10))
 (segment (start 74.676 76.708) (end 78.232 73.152) (width 0.5) (layer "B.Cu") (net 10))
 (segment (start 77.7 70.84) (end 77.7 70.83) (width 0.5) (layer "B.Cu") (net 10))
 (via (at 74.97 68.9) (size 0.8) (drill 0.4) (layers "F.Cu" "B.Cu") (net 3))
 (segment (start 74.921418 73.86) (end 76.03 73.86) (width 0.5) (layer "B.Cu") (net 3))
 (segment (start 74.97 68.9) (end 74.03 69.84) (width 0.5) (layer "B.Cu") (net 3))
 (segment (start 77.588 72.302) (end 78.584082 72.302) (width 0.5) (layer "B.Cu") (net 3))
 (segment (start 74.03 72.968582) (end 74.921418 73.86) (width 0.5) (layer "B.Cu") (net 3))
 (segment (start 74.97 68.9) (end 74.96 68.91) (width 0.5) (layer "B.Cu") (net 3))
 (segment (start 78.584082 72.302) (end 81.2 74.917918) (width 0.5) (layer "B.Cu") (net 3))
 (segment (start 74.03 69.84) (end 74.03 72.968582) (width 0.5) (layer "B.Cu") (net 3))
 (segment (start 76.03 73.86) (end 77.588 72.302) (width 0.5) (layer "B.Cu") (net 3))
 (segment (start 81.2 74.917918) (end 81.2 77.2) (width 0.5) (layer "B.Cu") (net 3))
 (segment (start 80.4445 72.757) (end 80.93905 72.757) (width 0.5) (layer "F.Cu") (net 7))
 (segment (start 82.18 71.51605) (end 82.17 69.17) (width 0.5) (layer "F.Cu") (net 7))
 (segment (start 80.93905 72.757) (end 82.18 71.51605) (width 0.5) (layer "F.Cu") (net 7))
 (segment (start 82.17 69.17) (end 82.18 69.21) (width 0.5) (layer "F.Cu") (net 7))
 (via (at 82.17 69.17) (size 0.8) (drill 0.4) (layers "F.Cu" "B.Cu") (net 7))
 (segment (start 80.4 69.6) (end 81.74 69.6) (width 0.5) (layer "B.Cu") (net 7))
 (segment (start 81.74 69.6) (end 82.17 69.17) (width 0.5) (layer "B.Cu") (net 7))
 (via (at 75.0205 72.757) (size 0.8) (drill 0.4) (layers "F.Cu" "B.Cu") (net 5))
 (segment (start 76.2 71.5775) (end 76.2 66.4) (width 0.5) (layer "B.Cu") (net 5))
 (segment (start 75.0205 72.757) (end 76.2 71.5775) (width 0.5) (layer "B.Cu") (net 5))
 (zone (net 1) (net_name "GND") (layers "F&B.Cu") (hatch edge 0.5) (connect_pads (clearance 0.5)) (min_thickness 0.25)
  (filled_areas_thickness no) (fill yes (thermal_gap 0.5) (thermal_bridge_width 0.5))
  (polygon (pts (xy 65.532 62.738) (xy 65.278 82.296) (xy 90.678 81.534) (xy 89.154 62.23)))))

